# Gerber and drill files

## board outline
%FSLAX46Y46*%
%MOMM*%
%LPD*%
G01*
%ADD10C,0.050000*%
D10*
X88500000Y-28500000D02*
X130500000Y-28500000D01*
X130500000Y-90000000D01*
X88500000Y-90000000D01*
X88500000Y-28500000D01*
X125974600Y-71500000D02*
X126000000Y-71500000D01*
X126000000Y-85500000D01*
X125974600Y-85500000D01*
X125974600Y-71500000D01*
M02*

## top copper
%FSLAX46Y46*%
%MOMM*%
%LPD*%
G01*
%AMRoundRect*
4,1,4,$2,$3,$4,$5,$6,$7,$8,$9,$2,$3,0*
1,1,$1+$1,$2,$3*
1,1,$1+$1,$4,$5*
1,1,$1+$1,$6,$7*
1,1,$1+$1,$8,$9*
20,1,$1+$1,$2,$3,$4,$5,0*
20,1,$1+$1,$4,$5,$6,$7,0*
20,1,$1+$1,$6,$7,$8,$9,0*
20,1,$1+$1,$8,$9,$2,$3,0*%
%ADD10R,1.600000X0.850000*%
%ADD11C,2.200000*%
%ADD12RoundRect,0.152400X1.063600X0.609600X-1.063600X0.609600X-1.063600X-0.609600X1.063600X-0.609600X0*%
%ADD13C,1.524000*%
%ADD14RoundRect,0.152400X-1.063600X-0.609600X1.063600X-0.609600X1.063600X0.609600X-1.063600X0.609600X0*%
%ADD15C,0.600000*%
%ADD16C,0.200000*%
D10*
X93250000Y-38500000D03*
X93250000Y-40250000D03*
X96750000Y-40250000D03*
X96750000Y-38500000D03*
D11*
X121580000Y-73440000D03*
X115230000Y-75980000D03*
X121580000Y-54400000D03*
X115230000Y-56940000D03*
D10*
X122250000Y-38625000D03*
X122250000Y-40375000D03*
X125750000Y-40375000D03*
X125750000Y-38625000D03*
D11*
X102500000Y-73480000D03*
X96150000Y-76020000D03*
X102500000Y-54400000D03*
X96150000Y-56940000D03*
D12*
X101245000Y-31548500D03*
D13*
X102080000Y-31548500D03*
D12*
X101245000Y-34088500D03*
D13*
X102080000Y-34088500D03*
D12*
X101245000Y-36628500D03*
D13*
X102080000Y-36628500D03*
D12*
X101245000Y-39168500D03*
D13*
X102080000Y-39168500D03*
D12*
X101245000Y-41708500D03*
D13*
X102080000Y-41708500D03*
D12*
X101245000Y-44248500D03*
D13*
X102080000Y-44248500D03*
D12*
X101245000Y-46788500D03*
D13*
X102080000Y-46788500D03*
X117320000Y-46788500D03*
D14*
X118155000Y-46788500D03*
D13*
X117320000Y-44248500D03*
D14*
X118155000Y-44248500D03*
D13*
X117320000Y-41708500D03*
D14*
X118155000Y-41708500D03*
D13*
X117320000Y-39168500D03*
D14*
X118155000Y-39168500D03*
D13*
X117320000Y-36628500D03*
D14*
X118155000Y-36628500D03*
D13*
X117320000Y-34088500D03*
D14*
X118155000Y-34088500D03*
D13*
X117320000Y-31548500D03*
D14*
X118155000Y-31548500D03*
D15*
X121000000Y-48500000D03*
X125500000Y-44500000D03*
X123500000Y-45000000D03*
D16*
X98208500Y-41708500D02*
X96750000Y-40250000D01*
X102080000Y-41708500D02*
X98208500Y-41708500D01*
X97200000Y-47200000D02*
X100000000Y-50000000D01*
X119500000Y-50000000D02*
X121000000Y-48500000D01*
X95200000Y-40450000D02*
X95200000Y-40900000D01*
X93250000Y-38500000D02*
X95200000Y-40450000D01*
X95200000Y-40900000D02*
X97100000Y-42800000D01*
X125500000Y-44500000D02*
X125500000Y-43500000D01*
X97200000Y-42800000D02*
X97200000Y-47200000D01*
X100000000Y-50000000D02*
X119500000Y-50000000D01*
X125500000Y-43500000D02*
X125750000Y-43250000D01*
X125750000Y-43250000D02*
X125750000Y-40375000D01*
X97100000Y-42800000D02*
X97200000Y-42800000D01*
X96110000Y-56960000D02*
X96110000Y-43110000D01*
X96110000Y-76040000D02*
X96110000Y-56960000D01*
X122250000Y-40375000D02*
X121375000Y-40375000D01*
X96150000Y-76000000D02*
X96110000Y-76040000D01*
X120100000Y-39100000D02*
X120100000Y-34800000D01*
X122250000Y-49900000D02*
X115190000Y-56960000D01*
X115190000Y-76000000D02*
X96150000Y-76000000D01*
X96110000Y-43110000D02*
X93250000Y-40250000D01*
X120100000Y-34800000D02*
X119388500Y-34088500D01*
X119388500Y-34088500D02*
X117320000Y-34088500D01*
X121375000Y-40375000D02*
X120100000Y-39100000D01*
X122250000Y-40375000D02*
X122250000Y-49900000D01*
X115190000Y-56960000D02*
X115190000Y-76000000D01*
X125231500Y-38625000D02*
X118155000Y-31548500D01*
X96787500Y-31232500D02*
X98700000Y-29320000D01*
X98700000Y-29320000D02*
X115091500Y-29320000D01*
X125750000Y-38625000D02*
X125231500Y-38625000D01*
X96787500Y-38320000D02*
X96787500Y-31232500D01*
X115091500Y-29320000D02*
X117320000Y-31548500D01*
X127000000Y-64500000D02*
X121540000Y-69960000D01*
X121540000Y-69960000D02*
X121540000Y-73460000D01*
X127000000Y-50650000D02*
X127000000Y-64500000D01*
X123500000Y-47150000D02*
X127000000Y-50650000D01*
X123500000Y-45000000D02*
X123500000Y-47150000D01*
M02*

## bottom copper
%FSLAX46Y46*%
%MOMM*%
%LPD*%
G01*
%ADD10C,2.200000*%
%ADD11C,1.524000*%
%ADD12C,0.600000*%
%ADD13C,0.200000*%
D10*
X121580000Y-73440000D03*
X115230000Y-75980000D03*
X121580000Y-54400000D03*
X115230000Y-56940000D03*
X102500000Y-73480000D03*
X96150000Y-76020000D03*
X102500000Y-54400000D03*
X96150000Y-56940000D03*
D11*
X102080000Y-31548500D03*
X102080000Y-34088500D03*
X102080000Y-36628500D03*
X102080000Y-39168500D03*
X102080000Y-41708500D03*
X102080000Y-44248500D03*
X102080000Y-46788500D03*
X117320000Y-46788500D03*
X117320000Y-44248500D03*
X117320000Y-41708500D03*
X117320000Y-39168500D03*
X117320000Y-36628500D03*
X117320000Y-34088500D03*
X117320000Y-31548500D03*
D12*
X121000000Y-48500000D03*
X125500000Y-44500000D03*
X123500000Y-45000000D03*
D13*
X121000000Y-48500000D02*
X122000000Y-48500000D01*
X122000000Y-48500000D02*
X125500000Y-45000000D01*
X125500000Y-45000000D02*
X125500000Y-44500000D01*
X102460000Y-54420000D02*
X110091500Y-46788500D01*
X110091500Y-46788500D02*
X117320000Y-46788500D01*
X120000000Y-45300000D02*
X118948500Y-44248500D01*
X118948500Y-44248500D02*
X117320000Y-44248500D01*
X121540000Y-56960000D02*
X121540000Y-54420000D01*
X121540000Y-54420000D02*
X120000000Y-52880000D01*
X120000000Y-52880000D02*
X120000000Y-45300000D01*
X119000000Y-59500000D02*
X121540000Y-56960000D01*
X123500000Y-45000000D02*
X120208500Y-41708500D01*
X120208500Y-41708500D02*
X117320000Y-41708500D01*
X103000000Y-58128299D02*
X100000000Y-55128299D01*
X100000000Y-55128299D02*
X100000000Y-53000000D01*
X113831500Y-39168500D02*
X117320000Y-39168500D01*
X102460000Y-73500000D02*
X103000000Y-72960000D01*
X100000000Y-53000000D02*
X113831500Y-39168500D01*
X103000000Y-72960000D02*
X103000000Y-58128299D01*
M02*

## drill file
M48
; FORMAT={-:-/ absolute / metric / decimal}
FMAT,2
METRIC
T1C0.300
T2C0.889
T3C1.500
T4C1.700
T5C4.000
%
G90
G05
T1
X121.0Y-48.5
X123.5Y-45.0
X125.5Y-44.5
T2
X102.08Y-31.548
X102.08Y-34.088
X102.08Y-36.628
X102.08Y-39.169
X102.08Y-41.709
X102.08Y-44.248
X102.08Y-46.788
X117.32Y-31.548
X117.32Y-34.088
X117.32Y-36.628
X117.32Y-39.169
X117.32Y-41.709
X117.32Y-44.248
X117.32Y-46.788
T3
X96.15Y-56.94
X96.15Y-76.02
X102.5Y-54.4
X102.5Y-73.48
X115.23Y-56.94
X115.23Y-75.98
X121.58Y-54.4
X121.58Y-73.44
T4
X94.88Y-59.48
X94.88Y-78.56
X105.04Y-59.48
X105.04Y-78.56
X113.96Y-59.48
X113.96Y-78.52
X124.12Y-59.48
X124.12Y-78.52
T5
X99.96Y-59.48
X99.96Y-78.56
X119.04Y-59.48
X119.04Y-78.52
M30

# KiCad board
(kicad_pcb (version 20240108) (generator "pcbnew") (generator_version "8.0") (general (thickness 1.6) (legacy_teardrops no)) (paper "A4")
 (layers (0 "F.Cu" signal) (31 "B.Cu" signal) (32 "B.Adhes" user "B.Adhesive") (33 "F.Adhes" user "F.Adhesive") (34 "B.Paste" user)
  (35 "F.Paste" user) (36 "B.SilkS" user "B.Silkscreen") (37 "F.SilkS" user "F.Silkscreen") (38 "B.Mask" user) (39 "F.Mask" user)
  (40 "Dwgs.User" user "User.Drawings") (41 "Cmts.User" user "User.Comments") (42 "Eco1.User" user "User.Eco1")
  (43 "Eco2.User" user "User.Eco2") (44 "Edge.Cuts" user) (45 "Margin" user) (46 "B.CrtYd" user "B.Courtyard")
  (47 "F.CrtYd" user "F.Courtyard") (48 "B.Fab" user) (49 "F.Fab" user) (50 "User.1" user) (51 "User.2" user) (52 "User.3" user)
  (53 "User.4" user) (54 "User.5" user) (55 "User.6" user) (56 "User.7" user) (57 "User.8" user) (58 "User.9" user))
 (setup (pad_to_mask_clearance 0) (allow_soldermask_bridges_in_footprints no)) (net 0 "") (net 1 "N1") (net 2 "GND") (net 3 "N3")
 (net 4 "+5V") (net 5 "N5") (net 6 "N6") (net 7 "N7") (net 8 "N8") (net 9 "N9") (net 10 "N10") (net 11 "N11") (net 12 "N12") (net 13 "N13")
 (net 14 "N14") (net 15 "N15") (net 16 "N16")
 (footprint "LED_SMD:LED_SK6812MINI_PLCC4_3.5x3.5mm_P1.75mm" (layer "F.Cu") (at 95 39.375)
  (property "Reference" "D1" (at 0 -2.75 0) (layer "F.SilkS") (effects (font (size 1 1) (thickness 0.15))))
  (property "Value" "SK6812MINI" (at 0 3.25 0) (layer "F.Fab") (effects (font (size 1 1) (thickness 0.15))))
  (pad "1" smd rect (at -1.75 -0.875) (size 1.6 0.85) (layers "F.Cu" "F.Paste" "F.Mask") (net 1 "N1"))
  (pad "2" smd rect (at -1.75 0.875) (size 1.6 0.85) (layers "F.Cu" "F.Paste" "F.Mask") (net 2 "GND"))
  (pad "3" smd rect (at 1.75 0.875) (size 1.6 0.85) (layers "F.Cu" "F.Paste" "F.Mask") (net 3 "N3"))
  (pad "4" smd rect (at 1.75 -0.875) (size 1.6 0.85) (layers "F.Cu" "F.Paste" "F.Mask") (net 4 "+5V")))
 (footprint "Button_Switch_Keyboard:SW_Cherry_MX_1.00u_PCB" (layer "F.Cu") (at 121.58 73.44)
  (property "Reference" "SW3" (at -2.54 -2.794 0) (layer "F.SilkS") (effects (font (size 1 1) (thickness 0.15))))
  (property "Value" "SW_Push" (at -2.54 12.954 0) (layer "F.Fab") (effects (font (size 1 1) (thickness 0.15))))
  (pad "" np_thru_hole circle (at -7.62 5.08) (size 1.7 1.7) (drill 1.7) (layers "*.Cu" "*.Mask"))
  (pad "" np_thru_hole circle (at -2.54 5.08) (size 4 4) (drill 4) (layers "*.Cu" "*.Mask"))
  (pad "" np_thru_hole circle (at 2.54 5.08) (size 1.7 1.7) (drill 1.7) (layers "*.Cu" "*.Mask"))
  (pad "1" thru_hole circle (at 0 0) (size 2.2 2.2) (drill 1.5) (layers "*.Cu" "*.Mask") (remove_unused_layers no) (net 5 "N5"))
  (pad "2" thru_hole circle (at -6.35 2.54) (size 2.2 2.2) (drill 1.5) (layers "*.Cu" "*.Mask") (remove_unused_layers no) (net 2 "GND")))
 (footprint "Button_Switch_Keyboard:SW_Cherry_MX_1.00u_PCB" (layer "F.Cu") (at 121.58 54.4)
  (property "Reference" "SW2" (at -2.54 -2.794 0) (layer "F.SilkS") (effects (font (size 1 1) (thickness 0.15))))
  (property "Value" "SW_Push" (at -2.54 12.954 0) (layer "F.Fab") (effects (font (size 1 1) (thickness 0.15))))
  (pad "" np_thru_hole circle (at -7.62 5.08) (size 1.7 1.7) (drill 1.7) (layers "*.Cu" "*.Mask"))
  (pad "" np_thru_hole circle (at -2.54 5.08) (size 4 4) (drill 4) (layers "*.Cu" "*.Mask"))
  (pad "" np_thru_hole circle (at 2.54 5.08) (size 1.7 1.7) (drill 1.7) (layers "*.Cu" "*.Mask"))
  (pad "1" thru_hole circle (at 0 0) (size 2.2 2.2) (drill 1.5) (layers "*.Cu" "*.Mask") (remove_unused_layers no) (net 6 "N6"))
  (pad "2" thru_hole circle (at -6.35 2.54) (size 2.2 2.2) (drill 1.5) (layers "*.Cu" "*.Mask") (remove_unused_layers no) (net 2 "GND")))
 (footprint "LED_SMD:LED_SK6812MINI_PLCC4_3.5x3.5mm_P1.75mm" (layer "F.Cu") (at 124 39.5)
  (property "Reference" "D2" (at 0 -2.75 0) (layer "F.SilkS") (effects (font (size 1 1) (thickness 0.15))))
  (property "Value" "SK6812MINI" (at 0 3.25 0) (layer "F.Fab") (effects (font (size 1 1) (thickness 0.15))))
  (pad "1" smd rect (at -1.75 -0.875) (size 1.6 0.85) (layers "F.Cu" "F.Paste" "F.Mask") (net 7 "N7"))
  (pad "2" smd rect (at -1.75 0.875) (size 1.6 0.85) (layers "F.Cu" "F.Paste" "F.Mask") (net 2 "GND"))
  (pad "3" smd rect (at 1.75 0.875) (size 1.6 0.85) (layers "F.Cu" "F.Paste" "F.Mask") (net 1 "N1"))
  (pad "4" smd rect (at 1.75 -0.875) (size 1.6 0.85) (layers "F.Cu" "F.Paste" "F.Mask") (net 4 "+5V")))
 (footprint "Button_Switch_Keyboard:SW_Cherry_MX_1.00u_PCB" (layer "F.Cu") (at 102.5 73.48)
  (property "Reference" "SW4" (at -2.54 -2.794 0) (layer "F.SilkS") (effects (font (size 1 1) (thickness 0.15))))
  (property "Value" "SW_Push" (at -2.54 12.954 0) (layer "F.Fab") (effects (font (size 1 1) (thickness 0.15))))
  (pad "" np_thru_hole circle (at -7.62 5.08) (size 1.7 1.7) (drill 1.7) (layers "*.Cu" "*.Mask"))
  (pad "" np_thru_hole circle (at -2.54 5.08) (size 4 4) (drill 4) (layers "*.Cu" "*.Mask"))
  (pad "" np_thru_hole circle (at 2.54 5.08) (size 1.7 1.7) (drill 1.7) (layers "*.Cu" "*.Mask"))
  (pad "1" thru_hole circle (at 0 0) (size 2.2 2.2) (drill 1.5) (layers "*.Cu" "*.Mask") (remove_unused_layers no) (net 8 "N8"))
  (pad "2" thru_hole circle (at -6.35 2.54) (size 2.2 2.2) (drill 1.5) (layers "*.Cu" "*.Mask") (remove_unused_layers no) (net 2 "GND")))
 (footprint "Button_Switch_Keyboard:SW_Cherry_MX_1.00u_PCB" (layer "F.Cu") (at 102.5 54.4)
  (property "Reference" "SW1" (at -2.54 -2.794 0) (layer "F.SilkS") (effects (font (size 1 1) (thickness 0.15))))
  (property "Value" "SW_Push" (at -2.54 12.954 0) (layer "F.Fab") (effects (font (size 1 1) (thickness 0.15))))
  (pad "" np_thru_hole circle (at -7.62 5.08) (size 1.7 1.7) (drill 1.7) (layers "*.Cu" "*.Mask"))
  (pad "" np_thru_hole circle (at -2.54 5.08) (size 4 4) (drill 4) (layers "*.Cu" "*.Mask"))
  (pad "" np_thru_hole circle (at 2.54 5.08) (size 1.7 1.7) (drill 1.7) (layers "*.Cu" "*.Mask"))
  (pad "1" thru_hole circle (at 0 0) (size 2.2 2.2) (drill 1.5) (layers "*.Cu" "*.Mask") (remove_unused_layers no) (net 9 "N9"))
  (pad "2" thru_hole circle (at -6.35 2.54) (size 2.2 2.2) (drill 1.5) (layers "*.Cu" "*.Mask") (remove_unused_layers no) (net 2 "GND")))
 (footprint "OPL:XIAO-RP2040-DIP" (layer "F.Cu") (at 109.7 39.1685)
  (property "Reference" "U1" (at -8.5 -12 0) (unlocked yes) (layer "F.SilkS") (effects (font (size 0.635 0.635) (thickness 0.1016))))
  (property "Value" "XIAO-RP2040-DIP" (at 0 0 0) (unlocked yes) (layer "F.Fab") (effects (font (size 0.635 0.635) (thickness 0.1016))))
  (pad "1" smd roundrect (at -8.455 -7.62 180) (size 2.432 1.524) (layers "F.Cu" "F.Mask") (roundrect_rratio 0.1) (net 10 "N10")
   (thermal_bridge_angle 45))
  (pad "1" thru_hole circle (at -7.62 -7.62 180) (size 1.524 1.524) (drill 0.889) (layers "*.Cu" "*.Mask") (remove_unused_layers no)
   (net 10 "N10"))
  (pad "2" smd roundrect (at -8.455 -5.08 180) (size 2.432 1.524) (layers "F.Cu" "F.Mask") (roundrect_rratio 0.1) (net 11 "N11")
   (thermal_bridge_angle 45))
  (pad "2" thru_hole circle (at -7.62 -5.08 180) (size 1.524 1.524) (drill 0.889) (layers "*.Cu" "*.Mask") (remove_unused_layers no)
   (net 11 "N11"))
  (pad "3" smd roundrect (at -8.455 -2.54 180) (size 2.432 1.524) (layers "F.Cu" "F.Mask") (roundrect_rratio 0.1) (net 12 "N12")
   (thermal_bridge_angle 45))
  (pad "3" thru_hole circle (at -7.62 -2.54 180) (size 1.524 1.524) (drill 0.889) (layers "*.Cu" "*.Mask") (remove_unused_layers no)
   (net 12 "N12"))
  (pad "4" smd roundrect (at -8.455 0 180) (size 2.432 1.524) (layers "F.Cu" "F.Mask") (roundrect_rratio 0.1) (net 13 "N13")
   (thermal_bridge_angle 45))
  (pad "4" thru_hole circle (at -7.62 0 180) (size 1.524 1.524) (drill 0.889) (layers "*.Cu" "*.Mask") (remove_unused_layers no)
   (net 13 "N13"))
  (pad "5" smd roundrect (at -8.455 2.54 180) (size 2.432 1.524) (layers "F.Cu" "F.Mask") (roundrect_rratio 0.1) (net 3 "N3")
   (thermal_bridge_angle 45))
  (pad "5" thru_hole circle (at -7.62 2.54 180) (size 1.524 1.524) (drill 0.889) (layers "*.Cu" "*.Mask") (remove_unused_layers no)
   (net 3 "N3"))
  (pad "6" smd roundrect (at -8.455 5.08 180) (size 2.432 1.524) (layers "F.Cu" "F.Mask") (roundrect_rratio 0.1) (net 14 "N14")
   (thermal_bridge_angle 45))
  (pad "6" thru_hole circle (at -7.62 5.08 180) (size 1.524 1.524) (drill 0.889) (layers "*.Cu" "*.Mask") (remove_unused_layers no)
   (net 14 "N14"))
  (pad "7" smd roundrect (at -8.455 7.62 180) (size 2.432 1.524) (layers "F.Cu" "F.Mask") (roundrect_rratio 0.1) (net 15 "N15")
   (thermal_bridge_angle 45))
  (pad "7" thru_hole circle (at -7.62 7.62 180) (size 1.524 1.524) (drill 0.889) (layers "*.Cu" "*.Mask") (remove_unused_layers no)
   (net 15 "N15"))
  (pad "8" thru_hole circle (at 7.62 7.62) (size 1.524 1.524) (drill 0.889) (layers "*.Cu" "*.Mask") (remove_unused_layers no) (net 9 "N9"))
  (pad "8" smd roundrect (at 8.455 7.62) (size 2.432 1.524) (layers "F.Cu" "F.Mask") (roundrect_rratio 0.1) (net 9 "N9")
   (thermal_bridge_angle 45))
  (pad "9" thru_hole circle (at 7.62 5.08) (size 1.524 1.524) (drill 0.889) (layers "*.Cu" "*.Mask") (remove_unused_layers no) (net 6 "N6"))
  (pad "9" smd roundrect (at 8.455 5.08) (size 2.432 1.524) (layers "F.Cu" "F.Mask") (roundrect_rratio 0.1) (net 6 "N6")
   (thermal_bridge_angle 45))
  (pad "10" thru_hole circle (at 7.62 2.54) (size 1.524 1.524) (drill 0.889) (layers "*.Cu" "*.Mask") (remove_unused_layers no) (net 5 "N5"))
  (pad "10" smd roundrect (at 8.455 2.54) (size 2.432 1.524) (layers "F.Cu" "F.Mask") (roundrect_rratio 0.1) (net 5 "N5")
   (thermal_bridge_angle 45))
  (pad "11" thru_hole circle (at 7.62 0) (size 1.524 1.524) (drill 0.889) (layers "*.Cu" "*.Mask") (remove_unused_layers no) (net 8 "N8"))
  (pad "11" smd roundrect (at 8.455 0) (size 2.432 1.524) (layers "F.Cu" "F.Mask") (roundrect_rratio 0.1) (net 8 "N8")
   (thermal_bridge_angle 45))
  (pad "12" thru_hole circle (at 7.62 -2.54) (size 1.524 1.524) (drill 0.889) (layers "*.Cu" "*.Mask") (remove_unused_layers no)
   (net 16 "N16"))
  (pad "12" smd roundrect (at 8.455 -2.54) (size 2.432 1.524) (layers "F.Cu" "F.Mask") (roundrect_rratio 0.1) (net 16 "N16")
   (thermal_bridge_angle 45))
  (pad "13" thru_hole circle (at 7.62 -5.08) (size 1.524 1.524) (drill 0.889) (layers "*.Cu" "*.Mask") (remove_unused_layers no)
   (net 2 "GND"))
  (pad "13" smd roundrect (at 8.455 -5.08) (size 2.432 1.524) (layers "F.Cu" "F.Mask") (roundrect_rratio 0.1) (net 2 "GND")
   (thermal_bridge_angle 45))
  (pad "14" thru_hole circle (at 7.62 -7.62) (size 1.524 1.524) (drill 0.889) (layers "*.Cu" "*.Mask") (remove_unused_layers no)
   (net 4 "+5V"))
  (pad "14" smd roundrect (at 8.455 -7.62) (size 2.432 1.524) (layers "F.Cu" "F.Mask") (roundrect_rratio 0.1) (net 4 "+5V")
   (thermal_bridge_angle 45)))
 (gr_rect (start 88.5 28.5) (end 130.5 90) (stroke (width 0.05) (type default)) (fill none) (layer "Edge.Cuts"))
 (gr_rect (start 125.9746 71.5) (end 126 85.5) (stroke (width 0.05) (type default)) (fill none) (layer "Edge.Cuts"))
 (segment (start 98.2085 41.7085) (end 96.75 40.25) (width 0.2) (layer "F.Cu") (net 3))
 (segment (start 102.08 41.7085) (end 98.2085 41.7085) (width 0.2) (layer "F.Cu") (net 3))
 (segment (start 97.2 47.2) (end 100 50) (width 0.2) (layer "F.Cu") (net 1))
 (segment (start 119.5 50) (end 121 48.5) (width 0.2) (layer "F.Cu") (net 1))
 (segment (start 95.2 40.45) (end 95.2 40.9) (width 0.2) (layer "F.Cu") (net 1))
 (segment (start 93.25 38.5) (end 95.2 40.45) (width 0.2) (layer "F.Cu") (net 1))
 (segment (start 95.2 40.9) (end 97.1 42.8) (width 0.2) (layer "F.Cu") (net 1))
 (segment (start 125.5 44.5) (end 125.5 43.5) (width 0.2) (layer "F.Cu") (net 1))
 (segment (start 97.2 42.8) (end 97.2 47.2) (width 0.2) (layer "F.Cu") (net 1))
 (segment (start 100 50) (end 119.5 50) (width 0.2) (layer "F.Cu") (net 1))
 (segment (start 125.5 43.5) (end 125.75 43.25) (width 0.2) (layer "F.Cu") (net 1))
 (segment (start 125.75 43.25) (end 125.75 40.375) (width 0.2) (layer "F.Cu") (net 1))
 (segment (start 97.1 42.8) (end 97.2 42.8) (width 0.2) (layer "F.Cu") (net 1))
 (via (at 121 48.5) (size 0.6) (drill 0.3) (layers "F.Cu" "B.Cu") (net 1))
 (via (at 125.5 44.5) (size 0.6) (drill 0.3) (layers "F.Cu" "B.Cu") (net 1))
 (segment (start 121 48.5) (end 122 48.5) (width 0.2) (layer "B.Cu") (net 1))
 (segment (start 122 48.5) (end 125.5 45) (width 0.2) (layer "B.Cu") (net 1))
 (segment (start 125.5 45) (end 125.5 44.5) (width 0.2) (layer "B.Cu") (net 1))
 (segment (start 96.11 56.96) (end 96.11 43.11) (width 0.2) (layer "F.Cu") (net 2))
 (segment (start 96.11 76.04) (end 96.11 56.96) (width 0.2) (layer "F.Cu") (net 2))
 (segment (start 122.25 40.375) (end 121.375 40.375) (width 0.2) (layer "F.Cu") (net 2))
 (segment (start 96.15 76) (end 96.11 76.04) (width 0.2) (layer "F.Cu") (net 2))
 (segment (start 120.1 39.1) (end 120.1 34.8) (width 0.2) (layer "F.Cu") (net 2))
 (segment (start 122.25 49.9) (end 115.19 56.96) (width 0.2) (layer "F.Cu") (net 2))
 (segment (start 115.19 76) (end 96.15 76) (width 0.2) (layer "F.Cu") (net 2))
 (segment (start 96.11 43.11) (end 93.25 40.25) (width 0.2) (layer "F.Cu") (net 2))
 (segment (start 120.1 34.8) (end 119.3885 34.0885) (width 0.2) (layer "F.Cu") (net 2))
 (segment (start 119.3885 34.0885) (end 117.32 34.0885) (width 0.2) (layer "F.Cu") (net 2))
 (segment (start 121.375 40.375) (end 120.1 39.1) (width 0.2) (layer "F.Cu") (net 2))
 (segment (start 122.25 40.375) (end 122.25 49.9) (width 0.2) (layer "F.Cu") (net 2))
 (segment (start 115.19 56.96) (end 115.19 76) (width 0.2) (layer "F.Cu") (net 2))
 (segment (start 125.2315 38.625) (end 118.155 31.5485) (width 0.2) (layer "F.Cu") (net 4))
 (segment (start 96.7875 31.2325) (end 98.7 29.32) (width 0.2) (layer "F.Cu") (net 4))
 (segment (start 98.7 29.32) (end 115.0915 29.32) (width 0.2) (layer "F.Cu") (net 4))
 (segment (start 125.75 38.625) (end 125.2315 38.625) (width 0.2) (layer "F.Cu") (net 4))
 (segment (start 96.7875 38.32) (end 96.7875 31.2325) (width 0.2) (layer "F.Cu") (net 4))
 (segment (start 115.0915 29.32) (end 117.32 31.5485) (width 0.2) (layer "F.Cu") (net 4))
 (segment (start 102.46 54.42) (end 110.0915 46.7885) (width 0.2) (layer "B.Cu") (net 9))
 (segment (start 110.0915 46.7885) (end 117.32 46.7885) (width 0.2) (layer "B.Cu") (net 9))
 (segment (start 120 45.3) (end 118.9485 44.2485) (width 0.2) (layer "B.Cu") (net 6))
 (segment (start 118.9485 44.2485) (end 117.32 44.2485) (width 0.2) (layer "B.Cu") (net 6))
 (segment (start 121.54 56.96) (end 121.54 54.42) (width 0.2) (layer "B.Cu") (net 6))
 (segment (start 121.54 54.42) (end 120 52.88) (width 0.2) (layer "B.Cu") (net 6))
 (segment (start 120 52.88) (end 120 45.3) (width 0.2) (layer "B.Cu") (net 6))
 (segment (start 119 59.5) (end 121.54 56.96) (width 0.2) (layer "B.Cu") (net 6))
 (segment (start 127 64.5) (end 121.54 69.96) (width 0.2) (layer "F.Cu") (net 5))
 (segment (start 121.54 69.96) (end 121.54 73.46) (width 0.2) (layer "F.Cu") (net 5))
 (segment (start 127 50.65) (end 127 64.5) (width 0.2) (layer "F.Cu") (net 5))
 (segment (start 123.5 47.15) (end 127 50.65) (width 0.2) (layer "F.Cu") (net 5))
 (segment (start 123.5 45) (end 123.5 47.15) (width 0.2) (layer "F.Cu") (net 5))
 (via (at 123.5 45) (size 0.6) (drill 0.3) (layers "F.Cu" "B.Cu") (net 5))
 (segment (start 123.5 45) (end 120.2085 41.7085) (width 0.2) (layer "B.Cu") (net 5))
 (segment (start 120.2085 41.7085) (end 117.32 41.7085) (width 0.2) (layer "B.Cu") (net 5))
 (segment (start 103 58.128299) (end 100 55.128299) (width 0.2) (layer "B.Cu") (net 8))
 (segment (start 100 55.128299) (end 100 53) (width 0.2) (layer "B.Cu") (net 8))
 (segment (start 113.8315 39.1685) (end 117.32 39.1685) (width 0.2) (layer "B.Cu") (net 8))
 (segment (start 102.46 73.5) (end 103 72.96) (width 0.2) (layer "B.Cu") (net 8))
 (segment (start 100 53) (end 113.8315 39.1685) (width 0.2) (layer "B.Cu") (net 8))
 (segment (start 103 72.96) (end 103 58.128299) (width 0.2) (layer "B.Cu") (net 8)))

